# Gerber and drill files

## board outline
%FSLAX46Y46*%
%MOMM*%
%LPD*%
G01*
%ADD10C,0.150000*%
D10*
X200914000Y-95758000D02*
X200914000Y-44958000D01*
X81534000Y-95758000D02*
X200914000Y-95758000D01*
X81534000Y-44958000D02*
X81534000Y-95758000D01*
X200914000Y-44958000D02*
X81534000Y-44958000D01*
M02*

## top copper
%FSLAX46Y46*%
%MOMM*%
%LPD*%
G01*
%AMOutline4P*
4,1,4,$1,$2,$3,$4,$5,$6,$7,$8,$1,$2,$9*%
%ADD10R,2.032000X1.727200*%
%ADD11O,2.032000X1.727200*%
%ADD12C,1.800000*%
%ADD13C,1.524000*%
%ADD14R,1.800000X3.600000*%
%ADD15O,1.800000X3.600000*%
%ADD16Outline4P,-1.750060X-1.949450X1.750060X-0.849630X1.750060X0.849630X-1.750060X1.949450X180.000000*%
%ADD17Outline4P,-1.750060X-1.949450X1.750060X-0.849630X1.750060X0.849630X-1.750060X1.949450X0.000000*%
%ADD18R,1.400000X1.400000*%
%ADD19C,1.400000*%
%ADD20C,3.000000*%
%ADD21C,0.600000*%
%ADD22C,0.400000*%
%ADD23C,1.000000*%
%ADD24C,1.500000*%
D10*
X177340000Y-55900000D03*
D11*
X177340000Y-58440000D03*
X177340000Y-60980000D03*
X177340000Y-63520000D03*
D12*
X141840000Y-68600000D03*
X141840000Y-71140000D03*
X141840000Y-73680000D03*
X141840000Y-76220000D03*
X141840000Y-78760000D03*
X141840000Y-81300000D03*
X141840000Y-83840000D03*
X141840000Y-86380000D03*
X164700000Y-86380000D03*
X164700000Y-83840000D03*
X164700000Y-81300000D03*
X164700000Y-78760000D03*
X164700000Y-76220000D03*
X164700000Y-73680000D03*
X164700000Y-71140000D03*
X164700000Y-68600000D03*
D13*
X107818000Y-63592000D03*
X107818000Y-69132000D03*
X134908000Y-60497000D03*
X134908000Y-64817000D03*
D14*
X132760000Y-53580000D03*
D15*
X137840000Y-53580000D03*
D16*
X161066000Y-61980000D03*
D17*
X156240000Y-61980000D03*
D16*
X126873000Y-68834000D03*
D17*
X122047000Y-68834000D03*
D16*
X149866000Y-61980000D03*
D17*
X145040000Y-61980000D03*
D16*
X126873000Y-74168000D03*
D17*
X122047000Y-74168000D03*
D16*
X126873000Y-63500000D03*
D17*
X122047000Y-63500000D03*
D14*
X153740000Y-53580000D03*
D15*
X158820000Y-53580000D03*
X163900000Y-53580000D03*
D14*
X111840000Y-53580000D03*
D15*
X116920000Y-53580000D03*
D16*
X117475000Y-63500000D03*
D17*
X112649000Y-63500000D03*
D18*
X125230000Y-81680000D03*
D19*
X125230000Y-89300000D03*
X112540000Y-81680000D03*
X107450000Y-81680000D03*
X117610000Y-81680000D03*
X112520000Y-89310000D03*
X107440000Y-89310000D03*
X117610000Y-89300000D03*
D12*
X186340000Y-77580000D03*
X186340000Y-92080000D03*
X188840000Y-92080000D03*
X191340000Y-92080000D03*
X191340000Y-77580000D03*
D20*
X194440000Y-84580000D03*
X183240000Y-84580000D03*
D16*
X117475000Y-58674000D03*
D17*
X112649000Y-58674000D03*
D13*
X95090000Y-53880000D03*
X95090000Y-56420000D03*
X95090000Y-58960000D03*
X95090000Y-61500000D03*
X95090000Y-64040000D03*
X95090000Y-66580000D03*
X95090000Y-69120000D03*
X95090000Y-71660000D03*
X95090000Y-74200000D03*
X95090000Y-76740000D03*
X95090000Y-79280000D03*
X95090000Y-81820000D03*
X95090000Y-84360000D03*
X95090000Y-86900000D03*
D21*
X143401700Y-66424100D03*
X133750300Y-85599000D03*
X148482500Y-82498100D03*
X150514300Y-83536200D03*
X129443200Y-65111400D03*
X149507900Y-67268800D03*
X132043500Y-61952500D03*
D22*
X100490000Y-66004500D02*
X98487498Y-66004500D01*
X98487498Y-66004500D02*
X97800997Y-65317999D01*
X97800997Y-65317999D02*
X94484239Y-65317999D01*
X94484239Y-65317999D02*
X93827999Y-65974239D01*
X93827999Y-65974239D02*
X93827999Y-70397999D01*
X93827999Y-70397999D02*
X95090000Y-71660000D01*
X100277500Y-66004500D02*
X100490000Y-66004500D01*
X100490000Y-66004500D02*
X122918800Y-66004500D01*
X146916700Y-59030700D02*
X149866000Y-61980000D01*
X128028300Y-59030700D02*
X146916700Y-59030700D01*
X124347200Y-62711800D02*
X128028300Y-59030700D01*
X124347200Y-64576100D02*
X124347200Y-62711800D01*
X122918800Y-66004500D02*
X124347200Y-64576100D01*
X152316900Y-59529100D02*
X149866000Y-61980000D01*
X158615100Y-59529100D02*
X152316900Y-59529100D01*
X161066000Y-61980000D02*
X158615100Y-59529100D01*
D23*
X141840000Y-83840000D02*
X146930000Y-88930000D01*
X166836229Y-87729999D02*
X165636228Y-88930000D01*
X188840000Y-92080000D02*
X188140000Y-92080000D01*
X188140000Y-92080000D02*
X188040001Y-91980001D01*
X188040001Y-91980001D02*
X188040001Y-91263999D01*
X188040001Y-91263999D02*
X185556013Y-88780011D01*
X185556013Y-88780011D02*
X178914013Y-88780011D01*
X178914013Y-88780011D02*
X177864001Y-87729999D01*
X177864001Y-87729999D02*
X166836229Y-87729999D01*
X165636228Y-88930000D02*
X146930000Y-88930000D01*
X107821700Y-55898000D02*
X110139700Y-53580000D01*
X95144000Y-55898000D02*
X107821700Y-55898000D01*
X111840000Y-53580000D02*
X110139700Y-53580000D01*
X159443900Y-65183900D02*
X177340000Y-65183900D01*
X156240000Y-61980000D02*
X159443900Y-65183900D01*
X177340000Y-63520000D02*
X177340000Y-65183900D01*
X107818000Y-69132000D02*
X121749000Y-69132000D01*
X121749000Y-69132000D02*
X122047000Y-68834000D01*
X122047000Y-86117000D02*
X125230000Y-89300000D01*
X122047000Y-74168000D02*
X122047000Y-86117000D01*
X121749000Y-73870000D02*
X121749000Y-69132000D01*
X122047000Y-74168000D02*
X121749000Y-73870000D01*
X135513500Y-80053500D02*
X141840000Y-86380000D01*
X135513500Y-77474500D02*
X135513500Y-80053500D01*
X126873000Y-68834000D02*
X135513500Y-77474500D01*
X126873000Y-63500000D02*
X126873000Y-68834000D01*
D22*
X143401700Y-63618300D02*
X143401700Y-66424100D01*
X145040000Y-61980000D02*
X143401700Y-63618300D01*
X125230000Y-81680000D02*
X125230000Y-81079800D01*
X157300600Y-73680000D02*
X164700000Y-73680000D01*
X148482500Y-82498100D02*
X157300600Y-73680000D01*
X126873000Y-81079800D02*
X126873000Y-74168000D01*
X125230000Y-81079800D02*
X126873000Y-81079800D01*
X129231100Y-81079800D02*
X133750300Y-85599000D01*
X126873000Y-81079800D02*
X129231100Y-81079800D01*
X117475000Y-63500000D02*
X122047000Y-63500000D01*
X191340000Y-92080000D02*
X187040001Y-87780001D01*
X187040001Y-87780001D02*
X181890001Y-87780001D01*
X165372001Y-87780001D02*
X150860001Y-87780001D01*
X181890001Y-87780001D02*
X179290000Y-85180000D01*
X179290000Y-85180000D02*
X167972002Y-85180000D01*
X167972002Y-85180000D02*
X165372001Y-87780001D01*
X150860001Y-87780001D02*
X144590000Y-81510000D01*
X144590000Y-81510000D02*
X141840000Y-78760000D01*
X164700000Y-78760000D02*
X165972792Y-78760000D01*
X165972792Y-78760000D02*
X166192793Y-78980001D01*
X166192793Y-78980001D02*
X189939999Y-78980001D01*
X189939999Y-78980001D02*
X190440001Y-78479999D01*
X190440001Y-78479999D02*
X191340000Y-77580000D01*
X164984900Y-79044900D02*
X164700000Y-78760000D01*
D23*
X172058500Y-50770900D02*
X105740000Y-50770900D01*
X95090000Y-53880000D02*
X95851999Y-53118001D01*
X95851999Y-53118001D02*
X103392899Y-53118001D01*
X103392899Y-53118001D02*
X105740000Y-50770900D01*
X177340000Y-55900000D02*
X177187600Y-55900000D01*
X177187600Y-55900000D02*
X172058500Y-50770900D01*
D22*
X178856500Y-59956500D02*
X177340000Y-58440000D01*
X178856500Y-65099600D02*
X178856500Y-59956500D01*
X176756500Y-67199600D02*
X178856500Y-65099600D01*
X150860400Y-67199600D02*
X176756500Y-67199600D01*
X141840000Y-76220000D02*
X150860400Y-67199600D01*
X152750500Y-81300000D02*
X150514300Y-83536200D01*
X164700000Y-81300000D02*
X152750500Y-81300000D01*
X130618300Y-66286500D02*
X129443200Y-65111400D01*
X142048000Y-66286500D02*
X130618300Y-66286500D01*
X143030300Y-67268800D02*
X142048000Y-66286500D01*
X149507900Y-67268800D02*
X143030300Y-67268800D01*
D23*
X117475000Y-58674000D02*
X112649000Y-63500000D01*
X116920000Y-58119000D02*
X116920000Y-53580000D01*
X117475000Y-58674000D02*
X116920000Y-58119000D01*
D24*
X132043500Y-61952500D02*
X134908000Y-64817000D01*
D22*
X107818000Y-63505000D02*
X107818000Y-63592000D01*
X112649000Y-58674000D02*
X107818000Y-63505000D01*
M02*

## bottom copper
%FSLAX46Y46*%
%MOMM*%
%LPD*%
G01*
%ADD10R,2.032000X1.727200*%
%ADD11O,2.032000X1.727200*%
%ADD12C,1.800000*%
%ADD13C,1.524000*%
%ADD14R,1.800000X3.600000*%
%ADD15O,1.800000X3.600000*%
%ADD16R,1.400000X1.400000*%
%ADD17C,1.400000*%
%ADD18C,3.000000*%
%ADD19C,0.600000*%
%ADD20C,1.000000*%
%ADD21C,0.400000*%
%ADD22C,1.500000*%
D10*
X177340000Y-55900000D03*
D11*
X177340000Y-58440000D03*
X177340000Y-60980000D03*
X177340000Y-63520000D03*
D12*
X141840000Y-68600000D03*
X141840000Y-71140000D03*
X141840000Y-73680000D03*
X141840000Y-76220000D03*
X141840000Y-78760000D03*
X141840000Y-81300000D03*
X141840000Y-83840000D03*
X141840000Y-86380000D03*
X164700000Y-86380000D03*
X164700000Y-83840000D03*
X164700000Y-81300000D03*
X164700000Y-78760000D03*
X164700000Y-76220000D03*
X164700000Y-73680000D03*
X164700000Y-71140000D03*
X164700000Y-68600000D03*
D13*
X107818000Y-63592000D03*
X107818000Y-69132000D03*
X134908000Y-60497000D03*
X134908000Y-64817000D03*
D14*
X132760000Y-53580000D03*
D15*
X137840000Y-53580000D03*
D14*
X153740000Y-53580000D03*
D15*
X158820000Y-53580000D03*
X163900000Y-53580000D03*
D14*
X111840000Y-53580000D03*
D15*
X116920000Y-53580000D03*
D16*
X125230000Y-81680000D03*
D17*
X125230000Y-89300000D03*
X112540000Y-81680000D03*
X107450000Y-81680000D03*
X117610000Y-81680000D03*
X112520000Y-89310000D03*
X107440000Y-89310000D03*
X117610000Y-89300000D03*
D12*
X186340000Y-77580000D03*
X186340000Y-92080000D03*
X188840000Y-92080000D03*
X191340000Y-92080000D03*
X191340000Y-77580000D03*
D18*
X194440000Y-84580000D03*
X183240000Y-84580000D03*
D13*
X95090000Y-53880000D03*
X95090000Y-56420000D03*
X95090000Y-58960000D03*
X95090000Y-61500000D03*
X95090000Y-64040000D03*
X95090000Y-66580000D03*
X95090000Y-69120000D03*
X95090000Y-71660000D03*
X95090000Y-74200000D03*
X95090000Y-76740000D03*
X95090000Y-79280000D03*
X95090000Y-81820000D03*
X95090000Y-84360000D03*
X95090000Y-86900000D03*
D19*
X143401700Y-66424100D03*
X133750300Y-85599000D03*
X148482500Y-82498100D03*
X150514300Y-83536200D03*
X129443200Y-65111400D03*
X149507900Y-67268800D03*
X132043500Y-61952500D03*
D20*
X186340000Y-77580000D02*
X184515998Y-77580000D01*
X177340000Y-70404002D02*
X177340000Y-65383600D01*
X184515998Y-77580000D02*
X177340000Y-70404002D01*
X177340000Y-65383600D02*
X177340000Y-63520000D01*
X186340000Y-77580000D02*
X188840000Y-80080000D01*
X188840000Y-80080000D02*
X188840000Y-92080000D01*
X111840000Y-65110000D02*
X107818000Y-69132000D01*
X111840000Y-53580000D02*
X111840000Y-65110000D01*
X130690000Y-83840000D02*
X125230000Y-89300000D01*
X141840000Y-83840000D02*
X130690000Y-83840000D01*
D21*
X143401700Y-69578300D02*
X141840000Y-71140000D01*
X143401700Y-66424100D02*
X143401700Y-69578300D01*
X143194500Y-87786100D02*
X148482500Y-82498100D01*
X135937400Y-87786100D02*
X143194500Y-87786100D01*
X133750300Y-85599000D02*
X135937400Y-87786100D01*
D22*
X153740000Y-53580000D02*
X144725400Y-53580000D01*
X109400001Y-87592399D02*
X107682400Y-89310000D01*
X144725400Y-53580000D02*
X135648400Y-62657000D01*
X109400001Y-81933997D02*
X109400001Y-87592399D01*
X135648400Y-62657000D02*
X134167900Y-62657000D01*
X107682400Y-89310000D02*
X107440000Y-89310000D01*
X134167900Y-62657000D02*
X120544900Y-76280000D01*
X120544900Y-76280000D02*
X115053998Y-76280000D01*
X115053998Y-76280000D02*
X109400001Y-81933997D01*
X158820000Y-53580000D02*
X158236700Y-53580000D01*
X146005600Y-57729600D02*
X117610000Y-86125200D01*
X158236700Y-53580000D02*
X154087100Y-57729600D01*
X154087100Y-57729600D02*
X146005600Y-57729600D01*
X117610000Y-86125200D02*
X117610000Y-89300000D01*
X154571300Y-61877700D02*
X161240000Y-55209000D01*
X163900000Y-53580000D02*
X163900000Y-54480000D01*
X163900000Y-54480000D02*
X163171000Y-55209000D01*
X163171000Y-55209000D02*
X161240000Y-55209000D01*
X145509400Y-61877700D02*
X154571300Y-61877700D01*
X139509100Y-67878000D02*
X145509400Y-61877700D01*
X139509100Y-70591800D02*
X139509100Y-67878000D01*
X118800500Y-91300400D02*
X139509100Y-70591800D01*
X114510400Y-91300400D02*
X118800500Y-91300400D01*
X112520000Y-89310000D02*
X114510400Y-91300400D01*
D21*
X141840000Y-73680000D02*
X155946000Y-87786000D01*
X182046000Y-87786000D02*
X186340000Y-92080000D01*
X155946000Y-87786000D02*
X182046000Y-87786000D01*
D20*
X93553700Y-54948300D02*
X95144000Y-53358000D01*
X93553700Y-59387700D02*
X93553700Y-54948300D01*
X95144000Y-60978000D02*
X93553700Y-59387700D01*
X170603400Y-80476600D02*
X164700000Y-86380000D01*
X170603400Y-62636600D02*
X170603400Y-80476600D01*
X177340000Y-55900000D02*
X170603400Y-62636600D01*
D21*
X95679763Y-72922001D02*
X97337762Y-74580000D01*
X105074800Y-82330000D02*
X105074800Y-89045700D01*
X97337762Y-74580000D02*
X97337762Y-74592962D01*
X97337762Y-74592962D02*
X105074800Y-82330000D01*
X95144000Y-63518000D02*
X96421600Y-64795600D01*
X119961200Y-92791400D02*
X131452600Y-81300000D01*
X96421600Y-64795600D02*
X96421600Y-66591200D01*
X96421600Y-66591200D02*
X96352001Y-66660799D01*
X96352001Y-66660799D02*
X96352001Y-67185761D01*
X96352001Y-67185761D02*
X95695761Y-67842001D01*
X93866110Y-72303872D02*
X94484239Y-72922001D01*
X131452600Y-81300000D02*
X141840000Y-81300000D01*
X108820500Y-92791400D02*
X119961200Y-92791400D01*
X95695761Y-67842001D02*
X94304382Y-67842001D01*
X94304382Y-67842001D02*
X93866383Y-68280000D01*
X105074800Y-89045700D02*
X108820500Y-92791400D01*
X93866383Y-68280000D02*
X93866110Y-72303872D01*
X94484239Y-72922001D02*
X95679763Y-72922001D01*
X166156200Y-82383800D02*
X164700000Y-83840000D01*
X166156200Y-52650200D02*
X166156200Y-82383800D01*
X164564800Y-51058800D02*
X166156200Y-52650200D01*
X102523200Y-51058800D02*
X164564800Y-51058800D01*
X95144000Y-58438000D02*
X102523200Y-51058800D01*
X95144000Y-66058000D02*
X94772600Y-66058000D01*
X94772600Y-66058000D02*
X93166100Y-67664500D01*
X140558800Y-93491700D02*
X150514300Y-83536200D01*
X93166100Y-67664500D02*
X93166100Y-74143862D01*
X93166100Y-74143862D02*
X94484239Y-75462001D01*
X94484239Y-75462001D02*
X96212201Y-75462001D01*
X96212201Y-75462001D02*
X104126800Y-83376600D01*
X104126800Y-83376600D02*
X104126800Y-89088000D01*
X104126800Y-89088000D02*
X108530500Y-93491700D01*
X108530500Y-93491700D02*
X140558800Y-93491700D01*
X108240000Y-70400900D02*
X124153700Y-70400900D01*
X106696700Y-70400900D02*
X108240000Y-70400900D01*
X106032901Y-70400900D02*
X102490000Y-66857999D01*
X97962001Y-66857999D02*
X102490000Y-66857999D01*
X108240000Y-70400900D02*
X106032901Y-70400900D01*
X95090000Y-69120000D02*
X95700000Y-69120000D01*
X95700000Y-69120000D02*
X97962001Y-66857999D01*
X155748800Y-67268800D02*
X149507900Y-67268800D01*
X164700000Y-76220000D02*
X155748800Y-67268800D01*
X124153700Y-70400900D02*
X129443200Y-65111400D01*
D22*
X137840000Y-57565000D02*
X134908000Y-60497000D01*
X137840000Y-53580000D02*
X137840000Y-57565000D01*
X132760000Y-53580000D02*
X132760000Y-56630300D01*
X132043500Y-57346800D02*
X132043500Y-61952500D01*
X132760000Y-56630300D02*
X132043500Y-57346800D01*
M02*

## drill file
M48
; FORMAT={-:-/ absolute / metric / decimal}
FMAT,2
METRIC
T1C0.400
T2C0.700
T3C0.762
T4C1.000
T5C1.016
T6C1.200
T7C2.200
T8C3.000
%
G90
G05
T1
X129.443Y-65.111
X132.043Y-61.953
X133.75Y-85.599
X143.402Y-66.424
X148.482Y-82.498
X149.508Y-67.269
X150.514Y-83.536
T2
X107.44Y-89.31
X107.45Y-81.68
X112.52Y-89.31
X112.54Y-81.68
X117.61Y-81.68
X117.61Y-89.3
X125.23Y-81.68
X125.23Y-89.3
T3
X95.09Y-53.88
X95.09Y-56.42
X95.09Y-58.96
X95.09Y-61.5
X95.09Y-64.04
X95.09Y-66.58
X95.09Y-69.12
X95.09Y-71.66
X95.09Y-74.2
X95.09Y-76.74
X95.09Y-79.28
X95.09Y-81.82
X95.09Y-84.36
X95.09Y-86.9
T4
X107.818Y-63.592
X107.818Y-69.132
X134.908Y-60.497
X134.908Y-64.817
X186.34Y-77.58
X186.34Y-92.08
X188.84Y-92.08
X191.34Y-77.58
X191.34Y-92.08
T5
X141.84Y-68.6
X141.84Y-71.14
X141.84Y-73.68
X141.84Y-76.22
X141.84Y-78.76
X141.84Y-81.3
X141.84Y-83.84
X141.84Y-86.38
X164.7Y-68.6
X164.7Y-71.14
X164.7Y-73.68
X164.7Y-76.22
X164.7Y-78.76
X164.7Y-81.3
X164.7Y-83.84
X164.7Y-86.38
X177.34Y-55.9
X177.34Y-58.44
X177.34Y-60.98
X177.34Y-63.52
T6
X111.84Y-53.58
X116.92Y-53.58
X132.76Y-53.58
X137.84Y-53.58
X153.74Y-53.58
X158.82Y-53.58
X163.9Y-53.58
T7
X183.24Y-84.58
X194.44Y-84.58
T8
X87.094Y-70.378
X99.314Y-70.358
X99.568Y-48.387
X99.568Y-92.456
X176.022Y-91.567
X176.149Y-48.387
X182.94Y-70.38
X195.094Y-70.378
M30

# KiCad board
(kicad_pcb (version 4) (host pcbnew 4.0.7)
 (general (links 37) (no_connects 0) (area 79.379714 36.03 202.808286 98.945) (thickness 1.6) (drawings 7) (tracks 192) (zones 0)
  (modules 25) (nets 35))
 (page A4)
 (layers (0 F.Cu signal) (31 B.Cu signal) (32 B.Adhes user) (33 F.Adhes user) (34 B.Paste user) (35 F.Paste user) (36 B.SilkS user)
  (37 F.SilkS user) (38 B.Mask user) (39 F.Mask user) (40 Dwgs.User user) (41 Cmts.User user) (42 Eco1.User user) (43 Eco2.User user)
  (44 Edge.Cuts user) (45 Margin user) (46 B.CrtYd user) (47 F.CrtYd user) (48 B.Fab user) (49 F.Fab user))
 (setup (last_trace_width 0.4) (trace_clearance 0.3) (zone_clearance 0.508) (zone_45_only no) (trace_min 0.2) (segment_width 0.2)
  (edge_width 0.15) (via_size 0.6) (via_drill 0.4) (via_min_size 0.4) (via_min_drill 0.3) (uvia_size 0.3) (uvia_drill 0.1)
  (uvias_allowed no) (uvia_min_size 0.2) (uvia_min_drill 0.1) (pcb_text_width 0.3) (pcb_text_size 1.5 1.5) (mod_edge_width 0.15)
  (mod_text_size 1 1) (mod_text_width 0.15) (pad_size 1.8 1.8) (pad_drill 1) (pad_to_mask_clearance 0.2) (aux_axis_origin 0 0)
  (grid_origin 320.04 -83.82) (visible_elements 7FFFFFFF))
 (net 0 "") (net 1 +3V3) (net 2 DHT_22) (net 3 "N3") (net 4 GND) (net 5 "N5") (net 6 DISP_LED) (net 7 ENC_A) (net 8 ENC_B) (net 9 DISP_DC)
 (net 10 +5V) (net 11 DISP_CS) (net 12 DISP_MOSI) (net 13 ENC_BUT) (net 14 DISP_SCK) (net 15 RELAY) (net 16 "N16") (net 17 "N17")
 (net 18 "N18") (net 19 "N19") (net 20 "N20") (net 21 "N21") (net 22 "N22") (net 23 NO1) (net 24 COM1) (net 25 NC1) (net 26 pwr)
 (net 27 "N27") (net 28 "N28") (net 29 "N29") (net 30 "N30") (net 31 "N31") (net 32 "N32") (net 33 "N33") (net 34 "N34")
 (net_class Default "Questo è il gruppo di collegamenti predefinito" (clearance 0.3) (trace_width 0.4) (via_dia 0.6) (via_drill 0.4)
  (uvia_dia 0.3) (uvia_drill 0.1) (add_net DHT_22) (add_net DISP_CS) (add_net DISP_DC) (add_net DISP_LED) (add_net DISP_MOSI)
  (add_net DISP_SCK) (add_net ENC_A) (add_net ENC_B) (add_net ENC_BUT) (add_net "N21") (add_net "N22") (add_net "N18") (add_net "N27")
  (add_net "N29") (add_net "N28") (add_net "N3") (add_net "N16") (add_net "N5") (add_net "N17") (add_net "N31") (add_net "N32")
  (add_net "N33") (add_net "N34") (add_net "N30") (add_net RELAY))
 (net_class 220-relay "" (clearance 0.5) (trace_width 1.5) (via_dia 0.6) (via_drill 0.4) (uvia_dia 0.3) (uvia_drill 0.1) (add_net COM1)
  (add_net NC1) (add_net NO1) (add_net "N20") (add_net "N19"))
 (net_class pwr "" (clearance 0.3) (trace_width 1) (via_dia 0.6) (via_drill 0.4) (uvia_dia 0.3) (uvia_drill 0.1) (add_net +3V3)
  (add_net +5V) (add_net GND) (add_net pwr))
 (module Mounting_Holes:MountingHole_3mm (layer F.Cu) (at 176.022 91.567 180)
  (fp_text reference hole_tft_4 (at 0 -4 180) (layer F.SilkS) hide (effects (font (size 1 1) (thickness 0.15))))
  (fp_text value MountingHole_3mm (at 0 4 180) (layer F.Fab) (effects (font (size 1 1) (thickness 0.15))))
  (pad 1 np_thru_hole circle (at 0 0 180) (size 3 3) (drill 3) (layers *.Cu *.Mask)))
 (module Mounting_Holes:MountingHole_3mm (layer F.Cu) (at 182.94 70.38 180)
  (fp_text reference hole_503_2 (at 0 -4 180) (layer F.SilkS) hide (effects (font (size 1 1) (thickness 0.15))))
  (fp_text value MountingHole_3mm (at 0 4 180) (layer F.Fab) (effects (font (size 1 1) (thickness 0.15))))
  (pad 1 np_thru_hole circle (at 0 0 180) (size 3 3) (drill 3) (layers *.Cu *.Mask)))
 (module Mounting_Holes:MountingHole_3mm (layer F.Cu) (at 176.149 48.387 180)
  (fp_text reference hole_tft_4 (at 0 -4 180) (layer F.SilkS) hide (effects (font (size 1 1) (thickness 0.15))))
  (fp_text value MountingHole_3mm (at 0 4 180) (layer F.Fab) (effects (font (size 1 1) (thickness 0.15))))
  (pad 1 np_thru_hole circle (at 0 0 180) (size 3 3) (drill 3) (layers *.Cu *.Mask)))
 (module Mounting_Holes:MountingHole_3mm (layer F.Cu) (at 99.568 48.387 180)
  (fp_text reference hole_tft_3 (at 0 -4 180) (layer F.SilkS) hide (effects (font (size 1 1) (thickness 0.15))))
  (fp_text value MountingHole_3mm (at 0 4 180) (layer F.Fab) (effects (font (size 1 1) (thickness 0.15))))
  (pad 1 np_thru_hole circle (at 0 0 180) (size 3 3) (drill 3) (layers *.Cu *.Mask)))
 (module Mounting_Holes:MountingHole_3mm (layer F.Cu) (at 99.568 92.456 180)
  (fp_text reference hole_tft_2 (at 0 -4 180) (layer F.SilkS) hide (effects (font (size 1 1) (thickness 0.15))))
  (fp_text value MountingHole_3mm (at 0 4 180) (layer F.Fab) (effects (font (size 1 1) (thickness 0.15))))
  (pad 1 np_thru_hole circle (at 0 0 180) (size 3 3) (drill 3) (layers *.Cu *.Mask)))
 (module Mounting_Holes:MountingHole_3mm (layer F.Cu) (at 87.094 70.378 180)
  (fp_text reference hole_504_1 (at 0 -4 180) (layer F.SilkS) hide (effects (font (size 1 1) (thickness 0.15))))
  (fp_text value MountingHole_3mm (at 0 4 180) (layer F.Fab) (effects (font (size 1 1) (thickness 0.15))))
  (pad 1 np_thru_hole circle (at 0 0 180) (size 3 3) (drill 3) (layers *.Cu *.Mask)))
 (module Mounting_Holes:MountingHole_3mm (layer F.Cu) (at 195.094 70.378 180)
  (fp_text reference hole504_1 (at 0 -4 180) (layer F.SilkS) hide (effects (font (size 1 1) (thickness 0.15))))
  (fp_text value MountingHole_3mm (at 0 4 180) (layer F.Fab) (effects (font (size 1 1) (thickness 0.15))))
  (pad 1 np_thru_hole circle (at 0 0 180) (size 3 3) (drill 3) (layers *.Cu *.Mask)))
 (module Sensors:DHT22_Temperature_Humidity (layer F.Cu) (at 177.34 59.71 270)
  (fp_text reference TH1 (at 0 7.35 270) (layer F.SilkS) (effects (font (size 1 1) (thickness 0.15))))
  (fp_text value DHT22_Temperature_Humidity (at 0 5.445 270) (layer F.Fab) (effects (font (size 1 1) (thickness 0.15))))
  (pad 1 thru_hole rect (at -3.81 0) (size 2.032 1.7272) (drill 1.016) (layers *.Cu *.Mask F.SilkS) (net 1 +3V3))
  (pad 2 thru_hole oval (at -1.27 0) (size 2.032 1.7272) (drill 1.016) (layers *.Cu *.Mask F.SilkS) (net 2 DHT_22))
  (pad 3 thru_hole oval (at 1.27 0) (size 2.032 1.7272) (drill 1.016) (layers *.Cu *.Mask F.SilkS) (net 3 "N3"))
  (pad 4 thru_hole oval (at 3.81 0) (size 2.032 1.7272) (drill 1.016) (layers *.Cu *.Mask F.SilkS) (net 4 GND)))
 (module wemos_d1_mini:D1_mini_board (layer F.Cu) (at 153.27 78.76)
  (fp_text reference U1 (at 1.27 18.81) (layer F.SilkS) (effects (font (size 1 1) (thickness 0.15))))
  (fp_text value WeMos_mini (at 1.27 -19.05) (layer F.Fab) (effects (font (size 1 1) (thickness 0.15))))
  (pad 8 thru_hole circle (at -11.43 -10.16) (size 1.8 1.8) (drill 1.016) (layers *.Cu *.Mask F.SilkS) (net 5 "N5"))
  (pad 7 thru_hole circle (at -11.43 -7.62) (size 1.8 1.8) (drill 1.016) (layers *.Cu *.Mask F.SilkS) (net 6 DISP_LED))
  (pad 6 thru_hole circle (at -11.43 -5.08) (size 1.8 1.8) (drill 1.016) (layers *.Cu *.Mask F.SilkS) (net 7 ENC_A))
  (pad 5 thru_hole circle (at -11.43 -2.54) (size 1.8 1.8) (drill 1.016) (layers *.Cu *.Mask F.SilkS) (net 2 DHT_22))
  (pad 4 thru_hole circle (at -11.43 0) (size 1.8 1.8) (drill 1.016) (layers *.Cu *.Mask F.SilkS) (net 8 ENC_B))
  (pad 3 thru_hole circle (at -11.43 2.54) (size 1.8 1.8) (drill 1.016) (layers *.Cu *.Mask F.SilkS) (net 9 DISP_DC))
  (pad 2 thru_hole circle (at -11.43 5.08) (size 1.8 1.8) (drill 1.016) (layers *.Cu *.Mask F.SilkS) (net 4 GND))
  (pad 1 thru_hole circle (at -11.43 7.62) (size 1.8 1.8) (drill 1.016) (layers *.Cu *.Mask F.SilkS) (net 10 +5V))
  (pad 16 thru_hole circle (at 11.43 7.62) (size 1.8 1.8) (drill 1.016) (layers *.Cu *.Mask F.SilkS) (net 1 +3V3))
  (pad 15 thru_hole circle (at 11.43 5.08) (size 1.8 1.8) (drill 1.016) (layers *.Cu *.Mask F.SilkS) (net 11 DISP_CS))
  (pad 14 thru_hole circle (at 11.43 2.54) (size 1.8 1.8) (drill 1.016) (layers *.Cu *.Mask F.SilkS) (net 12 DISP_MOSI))
  (pad 13 thru_hole circle (at 11.43 0) (size 1.8 1.8) (drill 1.016) (layers *.Cu *.Mask F.SilkS) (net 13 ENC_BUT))
  (pad 12 thru_hole circle (at 11.43 -2.54) (size 1.8 1.8) (drill 1.016) (layers *.Cu *.Mask F.SilkS) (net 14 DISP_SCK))
  (pad 11 thru_hole circle (at 11.43 -5.08) (size 1.8 1.8) (drill 1.016) (layers *.Cu *.Mask F.SilkS) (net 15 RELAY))
  (pad 10 thru_hole circle (at 11.43 -7.62) (size 1.8 1.8) (drill 1.016) (layers *.Cu *.Mask F.SilkS) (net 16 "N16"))
  (pad 9 thru_hole circle (at 11.43 -10.16) (size 1.8 1.8) (drill 1.016) (layers *.Cu *.Mask F.SilkS) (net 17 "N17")))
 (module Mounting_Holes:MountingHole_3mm (layer F.Cu) (at 99.314 70.358 180)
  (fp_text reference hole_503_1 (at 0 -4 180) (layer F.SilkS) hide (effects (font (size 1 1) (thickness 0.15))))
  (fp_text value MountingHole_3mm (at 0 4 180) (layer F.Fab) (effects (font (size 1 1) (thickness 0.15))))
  (pad 1 np_thru_hole circle (at 0 0 180) (size 3 3) (drill 3) (layers *.Cu *.Mask)))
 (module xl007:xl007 (layer F.Cu) (at 121.158 66.802)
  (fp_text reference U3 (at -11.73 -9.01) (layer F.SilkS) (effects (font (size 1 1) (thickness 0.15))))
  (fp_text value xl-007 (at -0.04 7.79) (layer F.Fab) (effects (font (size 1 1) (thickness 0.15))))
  (pad 3 thru_hole circle (at -13.34 -3.21) (size 1.524 1.524) (drill 1) (layers *.Cu *.Mask) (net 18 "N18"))
  (pad 4 thru_hole circle (at -13.34 2.33) (size 1.524 1.524) (drill 1) (layers *.Cu *.Mask) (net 4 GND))
  (pad 1 thru_hole circle (at 13.75 -6.305) (size 1.524 1.524) (drill 1) (layers *.Cu *.Mask) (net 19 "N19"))
  (pad 2 thru_hole circle (at 13.75 -1.985) (size 1.524 1.524) (drill 1) (layers *.Cu *.Mask) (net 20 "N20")))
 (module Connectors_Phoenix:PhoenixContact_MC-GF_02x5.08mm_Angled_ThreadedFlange (layer B.Cu) (at 132.76 53.58)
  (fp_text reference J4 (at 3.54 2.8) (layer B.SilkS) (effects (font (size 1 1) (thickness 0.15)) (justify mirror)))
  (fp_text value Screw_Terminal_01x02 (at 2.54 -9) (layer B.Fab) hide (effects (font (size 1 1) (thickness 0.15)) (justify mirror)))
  (pad 1 thru_hole rect (at 0 0) (size 1.8 3.6) (drill 1.2) (layers *.Cu *.Mask) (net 20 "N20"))
  (pad 2 thru_hole oval (at 5.08 0) (size 1.8 3.6) (drill 1.2) (layers *.Cu *.Mask) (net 19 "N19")))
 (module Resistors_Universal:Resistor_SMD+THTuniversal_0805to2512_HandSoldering (layer F.Cu) (at 158.653 61.98 180)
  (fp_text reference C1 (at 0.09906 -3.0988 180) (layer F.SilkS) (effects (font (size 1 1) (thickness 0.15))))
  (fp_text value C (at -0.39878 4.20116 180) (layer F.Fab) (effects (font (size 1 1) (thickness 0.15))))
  (pad 1 smd trapezoid (at -2.413 0 180) (size 3.50012 2.79908) (rect_delta 1.09982 0) (layers F.Cu F.Paste F.Mask) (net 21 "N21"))
  (pad 2 smd trapezoid (at 2.413 0) (size 3.50012 2.79908) (rect_delta 1.09982 0) (layers F.Cu F.Paste F.Mask) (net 4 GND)))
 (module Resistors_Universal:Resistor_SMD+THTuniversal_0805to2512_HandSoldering (layer F.Cu) (at 124.46 68.834 180)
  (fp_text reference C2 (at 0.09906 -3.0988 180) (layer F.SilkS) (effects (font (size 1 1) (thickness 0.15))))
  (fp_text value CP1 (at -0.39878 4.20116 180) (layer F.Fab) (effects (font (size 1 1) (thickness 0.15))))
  (pad 1 smd trapezoid (at -2.413 0 180) (size 3.50012 2.79908) (rect_delta 1.09982 0) (layers F.Cu F.Paste F.Mask) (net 10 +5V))
  (pad 2 smd trapezoid (at 2.413 0) (size 3.50012 2.79908) (rect_delta 1.09982 0) (layers F.Cu F.Paste F.Mask) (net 4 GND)))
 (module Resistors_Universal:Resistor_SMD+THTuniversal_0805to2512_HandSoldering (layer F.Cu) (at 147.453 61.98 180)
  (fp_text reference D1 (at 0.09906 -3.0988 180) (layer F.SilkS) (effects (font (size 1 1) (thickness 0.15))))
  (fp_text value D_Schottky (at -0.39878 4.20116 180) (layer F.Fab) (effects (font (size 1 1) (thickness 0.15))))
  (pad 1 smd trapezoid (at -2.413 0 180) (size 3.50012 2.79908) (rect_delta 1.09982 0) (layers F.Cu F.Paste F.Mask) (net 21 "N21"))
  (pad 2 smd trapezoid (at 2.413 0) (size 3.50012 2.79908) (rect_delta 1.09982 0) (layers F.Cu F.Paste F.Mask) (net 6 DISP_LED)))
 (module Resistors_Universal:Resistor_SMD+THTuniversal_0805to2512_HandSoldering (layer F.Cu) (at 124.46 74.168 180)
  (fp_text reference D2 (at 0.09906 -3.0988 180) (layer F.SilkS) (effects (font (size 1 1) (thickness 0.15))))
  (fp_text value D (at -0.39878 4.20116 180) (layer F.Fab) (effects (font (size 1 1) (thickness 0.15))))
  (pad 1 smd trapezoid (at -2.413 0 180) (size 3.50012 2.79908) (rect_delta 1.09982 0) (layers F.Cu F.Paste F.Mask) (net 15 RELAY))
  (pad 2 smd trapezoid (at 2.413 0) (size 3.50012 2.79908) (rect_delta 1.09982 0) (layers F.Cu F.Paste F.Mask) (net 4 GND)))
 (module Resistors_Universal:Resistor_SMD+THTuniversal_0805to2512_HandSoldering (layer F.Cu) (at 124.46 63.5 180)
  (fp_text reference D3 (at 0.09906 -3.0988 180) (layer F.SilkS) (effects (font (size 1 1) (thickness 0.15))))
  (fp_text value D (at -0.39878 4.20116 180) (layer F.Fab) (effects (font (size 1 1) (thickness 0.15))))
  (pad 1 smd trapezoid (at -2.413 0 180) (size 3.50012 2.79908) (rect_delta 1.09982 0) (layers F.Cu F.Paste F.Mask) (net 10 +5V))
  (pad 2 smd trapezoid (at 2.413 0) (size 3.50012 2.79908) (rect_delta 1.09982 0) (layers F.Cu F.Paste F.Mask) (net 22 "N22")))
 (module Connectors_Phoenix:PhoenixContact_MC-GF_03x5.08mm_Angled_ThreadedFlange (layer B.Cu) (at 153.74 53.58)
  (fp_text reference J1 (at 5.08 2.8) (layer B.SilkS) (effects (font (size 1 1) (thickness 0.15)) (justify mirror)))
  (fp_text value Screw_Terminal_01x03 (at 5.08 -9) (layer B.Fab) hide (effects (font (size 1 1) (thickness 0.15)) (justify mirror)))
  (pad 1 thru_hole rect (at 0 0) (size 1.8 3.6) (drill 1.2) (layers *.Cu *.Mask) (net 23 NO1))
  (pad 2 thru_hole oval (at 5.08 0) (size 1.8 3.6) (drill 1.2) (layers *.Cu *.Mask) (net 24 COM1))
  (pad 3 thru_hole oval (at 10.16 0) (size 1.8 3.6) (drill 1.2) (layers *.Cu *.Mask) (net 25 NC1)))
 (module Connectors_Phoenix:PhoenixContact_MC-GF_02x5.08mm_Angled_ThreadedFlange (layer B.Cu) (at 111.84 53.58)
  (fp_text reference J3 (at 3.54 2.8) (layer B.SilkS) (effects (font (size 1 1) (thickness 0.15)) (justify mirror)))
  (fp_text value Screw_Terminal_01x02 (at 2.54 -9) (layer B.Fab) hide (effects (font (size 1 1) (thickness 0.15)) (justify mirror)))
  (pad 1 thru_hole rect (at 0 0) (size 1.8 3.6) (drill 1.2) (layers *.Cu *.Mask) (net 4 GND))
  (pad 2 thru_hole oval (at 5.08 0) (size 1.8 3.6) (drill 1.2) (layers *.Cu *.Mask) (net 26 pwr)))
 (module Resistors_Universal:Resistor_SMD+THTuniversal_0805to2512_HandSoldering (layer F.Cu) (at 115.062 63.5 180)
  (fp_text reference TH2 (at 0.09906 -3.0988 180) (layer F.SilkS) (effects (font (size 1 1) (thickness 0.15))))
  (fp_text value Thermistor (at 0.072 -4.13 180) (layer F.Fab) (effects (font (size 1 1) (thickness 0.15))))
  (pad 1 smd trapezoid (at -2.413 0 180) (size 3.50012 2.79908) (rect_delta 1.09982 0) (layers F.Cu F.Paste F.Mask) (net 22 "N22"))
  (pad 2 smd trapezoid (at 2.413 0) (size 3.50012 2.79908) (rect_delta 1.09982 0) (layers F.Cu F.Paste F.Mask) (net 26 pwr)))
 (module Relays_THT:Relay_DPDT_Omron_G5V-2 (layer F.Cu) (at 125.23 81.68 270)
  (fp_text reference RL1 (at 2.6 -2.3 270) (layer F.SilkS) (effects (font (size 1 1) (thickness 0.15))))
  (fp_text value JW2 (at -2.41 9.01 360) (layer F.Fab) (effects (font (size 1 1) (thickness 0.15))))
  (pad 1 thru_hole rect (at 0 0 270) (size 1.4 1.4) (drill 0.7) (layers *.Cu *.Mask) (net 15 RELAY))
  (pad 8 thru_hole circle (at 7.62 0 270) (size 1.4 1.4) (drill 0.7) (layers *.Cu *.Mask) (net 4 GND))
  (pad 2 thru_hole circle (at 0 12.69 270) (size 1.4 1.4) (drill 0.7) (layers *.Cu *.Mask) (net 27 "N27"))
  (pad 4 thru_hole circle (at 0 17.78 270) (size 1.4 1.4) (drill 0.7) (layers *.Cu *.Mask) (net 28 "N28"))
  (pad 3 thru_hole circle (at 0 7.62 270) (size 1.4 1.4) (drill 0.7) (layers *.Cu *.Mask) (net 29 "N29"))
  (pad 7 thru_hole circle (at 7.63 12.71 270) (size 1.4 1.4) (drill 0.7) (layers *.Cu *.Mask) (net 25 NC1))
  (pad 5 thru_hole circle (at 7.63 17.79 270) (size 1.4 1.4) (drill 0.7) (layers *.Cu *.Mask) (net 23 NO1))
  (pad 6 thru_hole circle (at 7.62 7.62 270) (size 1.4 1.4) (drill 0.7) (layers *.Cu *.Mask) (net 24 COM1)))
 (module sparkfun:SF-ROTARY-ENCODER (layer F.Cu) (at 188.84 84.58)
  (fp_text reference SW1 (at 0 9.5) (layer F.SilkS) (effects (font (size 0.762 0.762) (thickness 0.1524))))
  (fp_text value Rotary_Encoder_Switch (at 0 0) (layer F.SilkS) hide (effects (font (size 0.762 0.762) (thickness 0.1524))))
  (pad 5 thru_hole circle (at -2.5 -7) (size 1.8 1.8) (drill 1) (layers *.Cu *.Mask F.SilkS) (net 4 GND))
  (pad 1 thru_hole circle (at -2.5 7.5) (size 1.8 1.8) (drill 1) (layers *.Cu *.Mask F.SilkS) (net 7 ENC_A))
  (pad 2 thru_hole circle (at 0 7.5) (size 1.8 1.8) (drill 1) (layers *.Cu *.Mask F.SilkS) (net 4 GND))
  (pad 3 thru_hole circle (at 2.5 7.5) (size 1.8 1.8) (drill 1) (layers *.Cu *.Mask F.SilkS) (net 8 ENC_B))
  (pad 4 thru_hole circle (at 2.5 -7) (size 1.8 1.8) (drill 1) (layers *.Cu *.Mask F.SilkS) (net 13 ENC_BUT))
  (pad "" thru_hole circle (at 5.6 0) (size 3 3) (drill 2.2) (layers *.Cu *.Mask F.SilkS))
  (pad "" thru_hole circle (at -5.6 0) (size 3 3) (drill 2.2) (layers *.Cu *.Mask F.SilkS)))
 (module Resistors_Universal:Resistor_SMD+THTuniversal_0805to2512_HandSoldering (layer F.Cu) (at 115.062 58.674 180)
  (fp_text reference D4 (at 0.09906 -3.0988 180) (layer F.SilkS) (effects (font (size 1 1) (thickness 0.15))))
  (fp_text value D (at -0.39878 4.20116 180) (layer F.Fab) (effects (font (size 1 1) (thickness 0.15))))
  (pad 1 smd trapezoid (at -2.413 0 180) (size 3.50012 2.79908) (rect_delta 1.09982 0) (layers F.Cu F.Paste F.Mask) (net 26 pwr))
  (pad 2 smd trapezoid (at 2.413 0) (size 3.50012 2.79908) (rect_delta 1.09982 0) (layers F.Cu F.Paste F.Mask) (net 18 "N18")))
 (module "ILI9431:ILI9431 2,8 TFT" (layer F.Cu) (at 136.09 70.38)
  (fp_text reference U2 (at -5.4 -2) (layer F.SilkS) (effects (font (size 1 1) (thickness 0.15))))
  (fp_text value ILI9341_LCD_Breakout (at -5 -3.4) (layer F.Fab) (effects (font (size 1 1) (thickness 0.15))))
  (pad 1 thru_hole circle (at -41 -16.5) (size 1.524 1.524) (drill 0.762) (layers *.Cu *.Mask) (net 1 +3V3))
  (pad 2 thru_hole circle (at -41 -13.96) (size 1.524 1.524) (drill 0.762) (layers *.Cu *.Mask) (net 4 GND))
  (pad 3 thru_hole circle (at -41 -11.42) (size 1.524 1.524) (drill 0.762) (layers *.Cu *.Mask) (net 11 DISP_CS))
  (pad 4 thru_hole circle (at -41 -8.88) (size 1.524 1.524) (drill 0.762) (layers *.Cu *.Mask) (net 1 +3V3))
  (pad 5 thru_hole circle (at -41 -6.34) (size 1.524 1.524) (drill 0.762) (layers *.Cu *.Mask) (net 9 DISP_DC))
  (pad 6 thru_hole circle (at -41 -3.8) (size 1.524 1.524) (drill 0.762) (layers *.Cu *.Mask) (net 12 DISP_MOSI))
  (pad 7 thru_hole circle (at -41 -1.26) (size 1.524 1.524) (drill 0.762) (layers *.Cu *.Mask) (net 14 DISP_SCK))
  (pad 8 thru_hole circle (at -41 1.28) (size 1.524 1.524) (drill 0.762) (layers *.Cu *.Mask) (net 21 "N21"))
  (pad 9 thru_hole circle (at -41 3.82) (size 1.524 1.524) (drill 0.762) (layers *.Cu *.Mask) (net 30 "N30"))
  (pad 10 thru_hole circle (at -41 6.36) (size 1.524 1.524) (drill 0.762) (layers *.Cu *.Mask) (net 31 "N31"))
  (pad 11 thru_hole circle (at -41 8.9) (size 1.524 1.524) (drill 0.762) (layers *.Cu *.Mask) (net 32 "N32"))
  (pad 12 thru_hole circle (at -41 11.44) (size 1.524 1.524) (drill 0.762) (layers *.Cu *.Mask) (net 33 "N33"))
  (pad 13 thru_hole circle (at -41 13.98) (size 1.524 1.524) (drill 0.762) (layers *.Cu *.Mask) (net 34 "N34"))
  (pad 14 thru_hole circle (at -41 16.52) (size 1.524 1.524) (drill 0.762) (layers *.Cu *.Mask)))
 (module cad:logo (layer B.Cu) (at 190.19 56.28 180)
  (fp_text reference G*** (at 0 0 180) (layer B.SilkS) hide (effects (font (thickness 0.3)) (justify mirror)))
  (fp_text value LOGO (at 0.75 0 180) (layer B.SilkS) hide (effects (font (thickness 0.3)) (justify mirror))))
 (gr_line (start 200.914 95.758) (end 200.914 44.958) (layer Edge.Cuts) (width 0.15))
 (gr_line (start 81.534 95.758) (end 200.914 95.758) (layer Edge.Cuts) (width 0.15))
 (gr_line (start 81.534 44.958) (end 81.534 95.758) (layer Edge.Cuts) (width 0.15))
 (gr_line (start 200.914 44.958) (end 81.534 44.958) (layer Edge.Cuts) (width 0.15))
 (segment (start 100.49 66.0045) (end 98.487498 66.0045) (width 0.4) (layer F.Cu) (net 21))
 (segment (start 98.487498 66.0045) (end 97.800997 65.317999) (width 0.4) (layer F.Cu) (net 21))
 (segment (start 97.800997 65.317999) (end 94.484239 65.317999) (width 0.4) (layer F.Cu) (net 21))
 (segment (start 94.484239 65.317999) (end 93.827999 65.974239) (width 0.4) (layer F.Cu) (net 21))
 (segment (start 93.827999 65.974239) (end 93.827999 70.397999) (width 0.4) (layer F.Cu) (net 21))
 (segment (start 93.827999 70.397999) (end 95.09 71.66) (width 0.4) (layer F.Cu) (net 21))
 (segment (start 100.2775 66.0045) (end 100.49 66.0045) (width 0.4) (layer F.Cu) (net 21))
 (segment (start 100.49 66.0045) (end 122.9188 66.0045) (width 0.4) (layer F.Cu) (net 21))
 (segment (start 146.9167 59.0307) (end 149.866 61.98) (width 0.4) (layer F.Cu) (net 21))
 (segment (start 128.0283 59.0307) (end 146.9167 59.0307) (width 0.4) (layer F.Cu) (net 21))
 (segment (start 124.3472 62.7118) (end 128.0283 59.0307) (width 0.4) (layer F.Cu) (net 21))
 (segment (start 124.3472 64.5761) (end 124.3472 62.7118) (width 0.4) (layer F.Cu) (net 21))
 (segment (start 122.9188 66.0045) (end 124.3472 64.5761) (width 0.4) (layer F.Cu) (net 21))
 (segment (start 152.3169 59.5291) (end 149.866 61.98) (width 0.4) (layer F.Cu) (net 21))
 (segment (start 158.6151 59.5291) (end 152.3169 59.5291) (width 0.4) (layer F.Cu) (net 21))
 (segment (start 161.066 61.98) (end 158.6151 59.5291) (width 0.4) (layer F.Cu) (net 21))
 (segment (start 141.84 83.84) (end 146.93 88.93) (width 1) (layer F.Cu) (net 4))
 (segment (start 166.836229 87.729999) (end 165.636228 88.93) (width 1) (layer F.Cu) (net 4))
 (segment (start 188.84 92.08) (end 188.14 92.08) (width 1) (layer F.Cu) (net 4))
 (segment (start 188.14 92.08) (end 188.040001 91.980001) (width 1) (layer F.Cu) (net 4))
 (segment (start 188.040001 91.980001) (end 188.040001 91.263999) (width 1) (layer F.Cu) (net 4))
 (segment (start 188.040001 91.263999) (end 185.556013 88.780011) (width 1) (layer F.Cu) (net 4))
 (segment (start 185.556013 88.780011) (end 178.914013 88.780011) (width 1) (layer F.Cu) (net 4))
 (segment (start 178.914013 88.780011) (end 177.864001 87.729999) (width 1) (layer F.Cu) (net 4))
 (segment (start 177.864001 87.729999) (end 166.836229 87.729999) (width 1) (layer F.Cu) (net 4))
 (segment (start 165.636228 88.93) (end 146.93 88.93) (width 1) (layer F.Cu) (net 4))
 (segment (start 186.34 77.58) (end 184.515998 77.58) (width 1) (layer B.Cu) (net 4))
 (segment (start 177.34 70.404002) (end 177.34 65.3836) (width 1) (layer B.Cu) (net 4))
 (segment (start 184.515998 77.58) (end 177.34 70.404002) (width 1) (layer B.Cu) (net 4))
 (segment (start 177.34 65.3836) (end 177.34 63.52) (width 1) (layer B.Cu) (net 4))
 (segment (start 186.34 77.58) (end 188.84 80.08) (width 1) (layer B.Cu) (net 4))
 (segment (start 188.84 80.08) (end 188.84 92.08) (width 1) (layer B.Cu) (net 4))
 (segment (start 107.8217 55.898) (end 110.1397 53.58) (width 1) (layer F.Cu) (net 4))
 (segment (start 95.144 55.898) (end 107.8217 55.898) (width 1) (layer F.Cu) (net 4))
 (segment (start 111.84 53.58) (end 110.1397 53.58) (width 1) (layer F.Cu) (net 4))
 (segment (start 159.4439 65.1839) (end 177.34 65.1839) (width 1) (layer F.Cu) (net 4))
 (segment (start 156.24 61.98) (end 159.4439 65.1839) (width 1) (layer F.Cu) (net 4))
 (segment (start 177.34 63.52) (end 177.34 65.1839) (width 1) (layer F.Cu) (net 4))
 (segment (start 111.84 65.11) (end 107.818 69.132) (width 1) (layer B.Cu) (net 4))
 (segment (start 111.84 53.58) (end 111.84 65.11) (width 1) (layer B.Cu) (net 4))
 (segment (start 130.69 83.84) (end 125.23 89.3) (width 1) (layer B.Cu) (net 4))
 (segment (start 141.84 83.84) (end 130.69 83.84) (width 1) (layer B.Cu) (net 4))
 (segment (start 107.818 69.132) (end 121.749 69.132) (width 1) (layer F.Cu) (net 4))
 (segment (start 121.749 69.132) (end 122.047 68.834) (width 1) (layer F.Cu) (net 4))
 (segment (start 122.047 86.117) (end 125.23 89.3) (width 1) (layer F.Cu) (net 4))
 (segment (start 122.047 74.168) (end 122.047 86.117) (width 1) (layer F.Cu) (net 4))
 (segment (start 121.749 73.87) (end 121.749 69.132) (width 1) (layer F.Cu) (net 4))
 (segment (start 122.047 74.168) (end 121.749 73.87) (width 1) (layer F.Cu) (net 4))
 (segment (start 135.5135 80.0535) (end 141.84 86.38) (width 1) (layer F.Cu) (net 10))
 (segment (start 135.5135 77.4745) (end 135.5135 80.0535) (width 1) (layer F.Cu) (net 10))
 (segment (start 126.873 68.834) (end 135.5135 77.4745) (width 1) (layer F.Cu) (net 10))
 (segment (start 126.873 63.5) (end 126.873 68.834) (width 1) (layer F.Cu) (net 10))
 (via (at 143.4017 66.4241) (size 0.6) (layers F.Cu B.Cu) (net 6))
 (segment (start 143.4017 63.6183) (end 143.4017 66.4241) (width 0.4) (layer F.Cu) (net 6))
 (segment (start 145.04 61.98) (end 143.4017 63.6183) (width 0.4) (layer F.Cu) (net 6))
 (segment (start 143.4017 69.5783) (end 141.84 71.14) (width 0.4) (layer B.Cu) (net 6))
 (segment (start 143.4017 66.4241) (end 143.4017 69.5783) (width 0.4) (layer B.Cu) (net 6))
 (via (at 133.7503 85.599) (size 0.6) (layers F.Cu B.Cu) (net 15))
 (via (at 148.4825 82.4981) (size 0.6) (layers F.Cu B.Cu) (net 15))
 (segment (start 125.23 81.68) (end 125.23 81.0798) (width 0.4) (layer F.Cu) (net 15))
 (segment (start 143.1945 87.7861) (end 148.4825 82.4981) (width 0.4) (layer B.Cu) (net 15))
 (segment (start 135.9374 87.7861) (end 143.1945 87.7861) (width 0.4) (layer B.Cu) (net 15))
 (segment (start 133.7503 85.599) (end 135.9374 87.7861) (width 0.4) (layer B.Cu) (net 15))
 (segment (start 157.3006 73.68) (end 164.7 73.68) (width 0.4) (layer F.Cu) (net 15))
 (segment (start 148.4825 82.4981) (end 157.3006 73.68) (width 0.4) (layer F.Cu) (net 15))
 (segment (start 126.873 81.0798) (end 126.873 74.168) (width 0.4) (layer F.Cu) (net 15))
 (segment (start 125.23 81.0798) (end 126.873 81.0798) (width 0.4) (layer F.Cu) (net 15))
 (segment (start 129.2311 81.0798) (end 133.7503 85.599) (width 0.4) (layer F.Cu) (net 15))
 (segment (start 126.873 81.0798) (end 129.2311 81.0798) (width 0.4) (layer F.Cu) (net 15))
 (segment (start 117.475 63.5) (end 122.047 63.5) (width 0.4) (layer F.Cu) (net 22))
 (segment (start 153.74 53.58) (end 144.7254 53.58) (width 1.5) (layer B.Cu) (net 23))
 (segment (start 109.400001 87.592399) (end 107.6824 89.31) (width 1.5) (layer B.Cu) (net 23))
 (segment (start 144.7254 53.58) (end 135.6484 62.657) (width 1.5) (layer B.Cu) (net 23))
 (segment (start 109.400001 81.933997) (end 109.400001 87.592399) (width 1.5) (layer B.Cu) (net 23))
 (segment (start 135.6484 62.657) (end 134.1679 62.657) (width 1.5) (layer B.Cu) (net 23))
 (segment (start 107.6824 89.31) (end 107.44 89.31) (width 1.5) (layer B.Cu) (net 23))
 (segment (start 134.1679 62.657) (end 120.5449 76.28) (width 1.5) (layer B.Cu) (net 23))
 (segment (start 120.5449 76.28) (end 115.053998 76.28) (width 1.5) (layer B.Cu) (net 23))
 (segment (start 115.053998 76.28) (end 109.400001 81.933997) (width 1.5) (layer B.Cu) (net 23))
 (segment (start 158.82 53.58) (end 158.2367 53.58) (width 1.5) (layer B.Cu) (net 24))
 (segment (start 146.0056 57.7296) (end 117.61 86.1252) (width 1.5) (layer B.Cu) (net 24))
 (segment (start 158.2367 53.58) (end 154.0871 57.7296) (width 1.5) (layer B.Cu) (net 24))
 (segment (start 154.0871 57.7296) (end 146.0056 57.7296) (width 1.5) (layer B.Cu) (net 24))
 (segment (start 117.61 86.1252) (end 117.61 89.3) (width 1.5) (layer B.Cu) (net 24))
 (segment (start 154.5713 61.8777) (end 161.24 55.209) (width 1.5) (layer B.Cu) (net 25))
 (segment (start 163.9 53.58) (end 163.9 54.48) (width 1.5) (layer B.Cu) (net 25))
 (segment (start 163.9 54.48) (end 163.171 55.209) (width 1.5) (layer B.Cu) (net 25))
 (segment (start 163.171 55.209) (end 161.24 55.209) (width 1.5) (layer B.Cu) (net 25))
 (segment (start 145.5094 61.8777) (end 154.5713 61.8777) (width 1.5) (layer B.Cu) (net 25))
 (segment (start 139.5091 67.878) (end 145.5094 61.8777) (width 1.5) (layer B.Cu) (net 25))
 (segment (start 139.5091 70.5918) (end 139.5091 67.878) (width 1.5) (layer B.Cu) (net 25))
 (segment (start 118.8005 91.3004) (end 139.5091 70.5918) (width 1.5) (layer B.Cu) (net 25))
 (segment (start 114.5104 91.3004) (end 118.8005 91.3004) (width 1.5) (layer B.Cu) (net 25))
 (segment (start 112.52 89.31) (end 114.5104 91.3004) (width 1.5) (layer B.Cu) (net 25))
 (segment (start 141.84 73.68) (end 155.946 87.786) (width 0.4) (layer B.Cu) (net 7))
 (segment (start 182.046 87.786) (end 186.34 92.08) (width 0.4) (layer B.Cu) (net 7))
 (segment (start 155.946 87.786) (end 182.046 87.786) (width 0.4) (layer B.Cu) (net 7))
 (segment (start 191.34 92.08) (end 187.040001 87.780001) (width 0.4) (layer F.Cu) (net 8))
 (segment (start 187.040001 87.780001) (end 181.890001 87.780001) (width 0.4) (layer F.Cu) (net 8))
 (segment (start 165.372001 87.780001) (end 150.860001 87.780001) (width 0.4) (layer F.Cu) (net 8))
 (segment (start 181.890001 87.780001) (end 179.29 85.18) (width 0.4) (layer F.Cu) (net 8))
 (segment (start 179.29 85.18) (end 167.972002 85.18) (width 0.4) (layer F.Cu) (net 8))
 (segment (start 167.972002 85.18) (end 165.372001 87.780001) (width 0.4) (layer F.Cu) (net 8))
 (segment (start 150.860001 87.780001) (end 144.59 81.51) (width 0.4) (layer F.Cu) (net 8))
 (segment (start 144.59 81.51) (end 141.84 78.76) (width 0.4) (layer F.Cu) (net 8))
 (segment (start 164.7 78.76) (end 165.972792 78.76) (width 0.4) (layer F.Cu) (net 13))
 (segment (start 165.972792 78.76) (end 166.192793 78.980001) (width 0.4) (layer F.Cu) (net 13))
 (segment (start 166.192793 78.980001) (end 189.939999 78.980001) (width 0.4) (layer F.Cu) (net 13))
 (segment (start 189.939999 78.980001) (end 190.440001 78.479999) (width 0.4) (layer F.Cu) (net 13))
 (segment (start 190.440001 78.479999) (end 191.34 77.58) (width 0.4) (layer F.Cu) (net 13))
 (segment (start 164.9849 79.0449) (end 164.7 78.76) (width 0.4) (layer F.Cu) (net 13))
 (segment (start 172.0585 50.7709) (end 105.74 50.7709) (width 1) (layer F.Cu) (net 1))
 (segment (start 95.09 53.88) (end 95.851999 53.118001) (width 1) (layer F.Cu) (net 1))
 (segment (start 95.851999 53.118001) (end 103.392899 53.118001) (width 1) (layer F.Cu) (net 1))
 (segment (start 103.392899 53.118001) (end 105.74 50.7709) (width 1) (layer F.Cu) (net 1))
 (segment (start 177.34 55.9) (end 177.1876 55.9) (width 1) (layer F.Cu) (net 1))
 (segment (start 177.1876 55.9) (end 172.0585 50.7709) (width 1) (layer F.Cu) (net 1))
 (segment (start 93.5537 54.9483) (end 95.144 53.358) (width 1) (layer B.Cu) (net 1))
 (segment (start 93.5537 59.3877) (end 93.5537 54.9483) (width 1) (layer B.Cu) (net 1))
 (segment (start 95.144 60.978) (end 93.5537 59.3877) (width 1) (layer B.Cu) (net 1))
 (segment (start 170.6034 80.4766) (end 164.7 86.38) (width 1) (layer B.Cu) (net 1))
 (segment (start 170.6034 62.6366) (end 170.6034 80.4766) (width 1) (layer B.Cu) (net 1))
 (segment (start 177.34 55.9) (end 170.6034 62.6366) (width 1) (layer B.Cu) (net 1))
 (segment (start 178.8565 59.9565) (end 177.34 58.44) (width 0.4) (layer F.Cu) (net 2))
 (segment (start 178.8565 65.0996) (end 178.8565 59.9565) (width 0.4) (layer F.Cu) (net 2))
 (segment (start 176.7565 67.1996) (end 178.8565 65.0996) (width 0.4) (layer F.Cu) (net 2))
 (segment (start 150.8604 67.1996) (end 176.7565 67.1996) (width 0.4) (layer F.Cu) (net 2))
 (segment (start 141.84 76.22) (end 150.8604 67.1996) (width 0.4) (layer F.Cu) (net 2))
 (segment (start 95.679763 72.922001) (end 97.337762 74.58) (width 0.4) (layer B.Cu) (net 9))
 (segment (start 105.0748 82.33) (end 105.0748 89.0457) (width 0.4) (layer B.Cu) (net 9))
 (segment (start 97.337762 74.58) (end 97.337762 74.592962) (width 0.4) (layer B.Cu) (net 9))
 (segment (start 97.337762 74.592962) (end 105.0748 82.33) (width 0.4) (layer B.Cu) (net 9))
 (segment (start 95.144 63.518) (end 96.4216 64.7956) (width 0.4) (layer B.Cu) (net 9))
 (segment (start 119.9612 92.7914) (end 131.4526 81.3) (width 0.4) (layer B.Cu) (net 9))
 (segment (start 96.4216 64.7956) (end 96.4216 66.5912) (width 0.4) (layer B.Cu) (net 9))
 (segment (start 96.4216 66.5912) (end 96.352001 66.660799) (width 0.4) (layer B.Cu) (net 9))
 (segment (start 96.352001 66.660799) (end 96.352001 67.185761) (width 0.4) (layer B.Cu) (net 9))
 (segment (start 96.352001 67.185761) (end 95.695761 67.842001) (width 0.4) (layer B.Cu) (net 9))
 (segment (start 93.86611 72.303872) (end 94.484239 72.922001) (width 0.4) (layer B.Cu) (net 9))
 (segment (start 131.4526 81.3) (end 141.84 81.3) (width 0.4) (layer B.Cu) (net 9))
 (segment (start 108.8205 92.7914) (end 119.9612 92.7914) (width 0.4) (layer B.Cu) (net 9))
 (segment (start 95.695761 67.842001) (end 94.304382 67.842001) (width 0.4) (layer B.Cu) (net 9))
 (segment (start 94.304382 67.842001) (end 93.866383 68.28) (width 0.4) (layer B.Cu) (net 9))
 (segment (start 105.0748 89.0457) (end 108.8205 92.7914) (width 0.4) (layer B.Cu) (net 9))
 (segment (start 93.866383 68.28) (end 93.86611 72.303872) (width 0.4) (layer B.Cu) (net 9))
 (segment (start 94.484239 72.922001) (end 95.679763 72.922001) (width 0.4) (layer B.Cu) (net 9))
 (segment (start 166.1562 82.3838) (end 164.7 83.84) (width 0.4) (layer B.Cu) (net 11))
 (segment (start 166.1562 52.6502) (end 166.1562 82.3838) (width 0.4) (layer B.Cu) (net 11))
 (segment (start 164.5648 51.0588) (end 166.1562 52.6502) (width 0.4) (layer B.Cu) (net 11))
 (segment (start 102.5232 51.0588) (end 164.5648 51.0588) (width 0.4) (layer B.Cu) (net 11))
 (segment (start 95.144 58.438) (end 102.5232 51.0588) (width 0.4) (layer B.Cu) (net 11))
 (segment (start 95.144 66.058) (end 94.7726 66.058) (width 0.4) (layer B.Cu) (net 12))
 (segment (start 94.7726 66.058) (end 93.1661 67.6645) (width 0.4) (layer B.Cu) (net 12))
 (segment (start 140.5588 93.4917) (end 150.5143 83.5362) (width 0.4) (layer B.Cu) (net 12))
 (segment (start 93.1661 67.6645) (end 93.1661 74.143862) (width 0.4) (layer B.Cu) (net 12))
 (segment (start 93.1661 74.143862) (end 94.484239 75.462001) (width 0.4) (layer B.Cu) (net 12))
 (segment (start 94.484239 75.462001) (end 96.212201 75.462001) (width 0.4) (layer B.Cu) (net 12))
 (segment (start 96.212201 75.462001) (end 104.1268 83.3766) (width 0.4) (layer B.Cu) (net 12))
 (segment (start 104.1268 83.3766) (end 104.1268 89.088) (width 0.4) (layer B.Cu) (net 12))
 (segment (start 104.1268 89.088) (end 108.5305 93.4917) (width 0.4) (layer B.Cu) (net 12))
 (segment (start 108.5305 93.4917) (end 140.5588 93.4917) (width 0.4) (layer B.Cu) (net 12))
 (via (at 150.5143 83.5362) (size 0.6) (layers F.Cu B.Cu) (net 12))
 (segment (start 152.7505 81.3) (end 150.5143 83.5362) (width 0.4) (layer F.Cu) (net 12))
 (segment (start 164.7 81.3) (end 152.7505 81.3) (width 0.4) (layer F.Cu) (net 12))
 (segment (start 108.24 70.4009) (end 124.1537 70.4009) (width 0.4) (layer B.Cu) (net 14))
 (segment (start 106.6967 70.4009) (end 108.24 70.4009) (width 0.4) (layer B.Cu) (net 14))
 (segment (start 106.032901 70.4009) (end 102.49 66.857999) (width 0.4) (layer B.Cu) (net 14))
 (segment (start 97.962001 66.857999) (end 102.49 66.857999) (width 0.4) (layer B.Cu) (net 14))
 (segment (start 108.24 70.4009) (end 106.032901 70.4009) (width 0.4) (layer B.Cu) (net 14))
 (segment (start 95.09 69.12) (end 95.7 69.12) (width 0.4) (layer B.Cu) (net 14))
 (segment (start 95.7 69.12) (end 97.962001 66.857999) (width 0.4) (layer B.Cu) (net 14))
 (via (at 129.4432 65.1114) (size 0.6) (layers F.Cu B.Cu) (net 14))
 (via (at 149.5079 67.2688) (size 0.6) (layers F.Cu B.Cu) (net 14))
 (segment (start 155.7488 67.2688) (end 149.5079 67.2688) (width 0.4) (layer B.Cu) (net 14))
 (segment (start 164.7 76.22) (end 155.7488 67.2688) (width 0.4) (layer B.Cu) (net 14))
 (segment (start 124.1537 70.4009) (end 129.4432 65.1114) (width 0.4) (layer B.Cu) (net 14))
 (segment (start 130.6183 66.2865) (end 129.4432 65.1114) (width 0.4) (layer F.Cu) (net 14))
 (segment (start 142.048 66.2865) (end 130.6183 66.2865) (width 0.4) (layer F.Cu) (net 14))
 (segment (start 143.0303 67.2688) (end 142.048 66.2865) (width 0.4) (layer F.Cu) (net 14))
 (segment (start 149.5079 67.2688) (end 143.0303 67.2688) (width 0.4) (layer F.Cu) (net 14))
 (segment (start 117.475 58.674) (end 112.649 63.5) (width 1) (layer F.Cu) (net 26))
 (segment (start 116.92 58.119) (end 116.92 53.58) (width 1) (layer F.Cu) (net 26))
 (segment (start 117.475 58.674) (end 116.92 58.119) (width 1) (layer F.Cu) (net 26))
 (segment (start 137.84 57.565) (end 134.908 60.497) (width 1.5) (layer B.Cu) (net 19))
 (segment (start 137.84 53.58) (end 137.84 57.565) (width 1.5) (layer B.Cu) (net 19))
 (via (at 132.0435 61.9525) (size 0.6) (layers F.Cu B.Cu) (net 20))
 (segment (start 132.76 53.58) (end 132.76 56.6303) (width 1.5) (layer B.Cu) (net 20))
 (segment (start 132.0435 57.3468) (end 132.0435 61.9525) (width 1.5) (layer B.Cu) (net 20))
 (segment (start 132.76 56.6303) (end 132.0435 57.3468) (width 1.5) (layer B.Cu) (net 20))
 (segment (start 132.0435 61.9525) (end 134.908 64.817) (width 1.5) (layer F.Cu) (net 20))
 (segment (start 107.818 63.505) (end 107.818 63.592) (width 0.4) (layer F.Cu) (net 18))
 (segment (start 112.649 58.674) (end 107.818 63.505) (width 0.4) (layer F.Cu) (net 18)))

